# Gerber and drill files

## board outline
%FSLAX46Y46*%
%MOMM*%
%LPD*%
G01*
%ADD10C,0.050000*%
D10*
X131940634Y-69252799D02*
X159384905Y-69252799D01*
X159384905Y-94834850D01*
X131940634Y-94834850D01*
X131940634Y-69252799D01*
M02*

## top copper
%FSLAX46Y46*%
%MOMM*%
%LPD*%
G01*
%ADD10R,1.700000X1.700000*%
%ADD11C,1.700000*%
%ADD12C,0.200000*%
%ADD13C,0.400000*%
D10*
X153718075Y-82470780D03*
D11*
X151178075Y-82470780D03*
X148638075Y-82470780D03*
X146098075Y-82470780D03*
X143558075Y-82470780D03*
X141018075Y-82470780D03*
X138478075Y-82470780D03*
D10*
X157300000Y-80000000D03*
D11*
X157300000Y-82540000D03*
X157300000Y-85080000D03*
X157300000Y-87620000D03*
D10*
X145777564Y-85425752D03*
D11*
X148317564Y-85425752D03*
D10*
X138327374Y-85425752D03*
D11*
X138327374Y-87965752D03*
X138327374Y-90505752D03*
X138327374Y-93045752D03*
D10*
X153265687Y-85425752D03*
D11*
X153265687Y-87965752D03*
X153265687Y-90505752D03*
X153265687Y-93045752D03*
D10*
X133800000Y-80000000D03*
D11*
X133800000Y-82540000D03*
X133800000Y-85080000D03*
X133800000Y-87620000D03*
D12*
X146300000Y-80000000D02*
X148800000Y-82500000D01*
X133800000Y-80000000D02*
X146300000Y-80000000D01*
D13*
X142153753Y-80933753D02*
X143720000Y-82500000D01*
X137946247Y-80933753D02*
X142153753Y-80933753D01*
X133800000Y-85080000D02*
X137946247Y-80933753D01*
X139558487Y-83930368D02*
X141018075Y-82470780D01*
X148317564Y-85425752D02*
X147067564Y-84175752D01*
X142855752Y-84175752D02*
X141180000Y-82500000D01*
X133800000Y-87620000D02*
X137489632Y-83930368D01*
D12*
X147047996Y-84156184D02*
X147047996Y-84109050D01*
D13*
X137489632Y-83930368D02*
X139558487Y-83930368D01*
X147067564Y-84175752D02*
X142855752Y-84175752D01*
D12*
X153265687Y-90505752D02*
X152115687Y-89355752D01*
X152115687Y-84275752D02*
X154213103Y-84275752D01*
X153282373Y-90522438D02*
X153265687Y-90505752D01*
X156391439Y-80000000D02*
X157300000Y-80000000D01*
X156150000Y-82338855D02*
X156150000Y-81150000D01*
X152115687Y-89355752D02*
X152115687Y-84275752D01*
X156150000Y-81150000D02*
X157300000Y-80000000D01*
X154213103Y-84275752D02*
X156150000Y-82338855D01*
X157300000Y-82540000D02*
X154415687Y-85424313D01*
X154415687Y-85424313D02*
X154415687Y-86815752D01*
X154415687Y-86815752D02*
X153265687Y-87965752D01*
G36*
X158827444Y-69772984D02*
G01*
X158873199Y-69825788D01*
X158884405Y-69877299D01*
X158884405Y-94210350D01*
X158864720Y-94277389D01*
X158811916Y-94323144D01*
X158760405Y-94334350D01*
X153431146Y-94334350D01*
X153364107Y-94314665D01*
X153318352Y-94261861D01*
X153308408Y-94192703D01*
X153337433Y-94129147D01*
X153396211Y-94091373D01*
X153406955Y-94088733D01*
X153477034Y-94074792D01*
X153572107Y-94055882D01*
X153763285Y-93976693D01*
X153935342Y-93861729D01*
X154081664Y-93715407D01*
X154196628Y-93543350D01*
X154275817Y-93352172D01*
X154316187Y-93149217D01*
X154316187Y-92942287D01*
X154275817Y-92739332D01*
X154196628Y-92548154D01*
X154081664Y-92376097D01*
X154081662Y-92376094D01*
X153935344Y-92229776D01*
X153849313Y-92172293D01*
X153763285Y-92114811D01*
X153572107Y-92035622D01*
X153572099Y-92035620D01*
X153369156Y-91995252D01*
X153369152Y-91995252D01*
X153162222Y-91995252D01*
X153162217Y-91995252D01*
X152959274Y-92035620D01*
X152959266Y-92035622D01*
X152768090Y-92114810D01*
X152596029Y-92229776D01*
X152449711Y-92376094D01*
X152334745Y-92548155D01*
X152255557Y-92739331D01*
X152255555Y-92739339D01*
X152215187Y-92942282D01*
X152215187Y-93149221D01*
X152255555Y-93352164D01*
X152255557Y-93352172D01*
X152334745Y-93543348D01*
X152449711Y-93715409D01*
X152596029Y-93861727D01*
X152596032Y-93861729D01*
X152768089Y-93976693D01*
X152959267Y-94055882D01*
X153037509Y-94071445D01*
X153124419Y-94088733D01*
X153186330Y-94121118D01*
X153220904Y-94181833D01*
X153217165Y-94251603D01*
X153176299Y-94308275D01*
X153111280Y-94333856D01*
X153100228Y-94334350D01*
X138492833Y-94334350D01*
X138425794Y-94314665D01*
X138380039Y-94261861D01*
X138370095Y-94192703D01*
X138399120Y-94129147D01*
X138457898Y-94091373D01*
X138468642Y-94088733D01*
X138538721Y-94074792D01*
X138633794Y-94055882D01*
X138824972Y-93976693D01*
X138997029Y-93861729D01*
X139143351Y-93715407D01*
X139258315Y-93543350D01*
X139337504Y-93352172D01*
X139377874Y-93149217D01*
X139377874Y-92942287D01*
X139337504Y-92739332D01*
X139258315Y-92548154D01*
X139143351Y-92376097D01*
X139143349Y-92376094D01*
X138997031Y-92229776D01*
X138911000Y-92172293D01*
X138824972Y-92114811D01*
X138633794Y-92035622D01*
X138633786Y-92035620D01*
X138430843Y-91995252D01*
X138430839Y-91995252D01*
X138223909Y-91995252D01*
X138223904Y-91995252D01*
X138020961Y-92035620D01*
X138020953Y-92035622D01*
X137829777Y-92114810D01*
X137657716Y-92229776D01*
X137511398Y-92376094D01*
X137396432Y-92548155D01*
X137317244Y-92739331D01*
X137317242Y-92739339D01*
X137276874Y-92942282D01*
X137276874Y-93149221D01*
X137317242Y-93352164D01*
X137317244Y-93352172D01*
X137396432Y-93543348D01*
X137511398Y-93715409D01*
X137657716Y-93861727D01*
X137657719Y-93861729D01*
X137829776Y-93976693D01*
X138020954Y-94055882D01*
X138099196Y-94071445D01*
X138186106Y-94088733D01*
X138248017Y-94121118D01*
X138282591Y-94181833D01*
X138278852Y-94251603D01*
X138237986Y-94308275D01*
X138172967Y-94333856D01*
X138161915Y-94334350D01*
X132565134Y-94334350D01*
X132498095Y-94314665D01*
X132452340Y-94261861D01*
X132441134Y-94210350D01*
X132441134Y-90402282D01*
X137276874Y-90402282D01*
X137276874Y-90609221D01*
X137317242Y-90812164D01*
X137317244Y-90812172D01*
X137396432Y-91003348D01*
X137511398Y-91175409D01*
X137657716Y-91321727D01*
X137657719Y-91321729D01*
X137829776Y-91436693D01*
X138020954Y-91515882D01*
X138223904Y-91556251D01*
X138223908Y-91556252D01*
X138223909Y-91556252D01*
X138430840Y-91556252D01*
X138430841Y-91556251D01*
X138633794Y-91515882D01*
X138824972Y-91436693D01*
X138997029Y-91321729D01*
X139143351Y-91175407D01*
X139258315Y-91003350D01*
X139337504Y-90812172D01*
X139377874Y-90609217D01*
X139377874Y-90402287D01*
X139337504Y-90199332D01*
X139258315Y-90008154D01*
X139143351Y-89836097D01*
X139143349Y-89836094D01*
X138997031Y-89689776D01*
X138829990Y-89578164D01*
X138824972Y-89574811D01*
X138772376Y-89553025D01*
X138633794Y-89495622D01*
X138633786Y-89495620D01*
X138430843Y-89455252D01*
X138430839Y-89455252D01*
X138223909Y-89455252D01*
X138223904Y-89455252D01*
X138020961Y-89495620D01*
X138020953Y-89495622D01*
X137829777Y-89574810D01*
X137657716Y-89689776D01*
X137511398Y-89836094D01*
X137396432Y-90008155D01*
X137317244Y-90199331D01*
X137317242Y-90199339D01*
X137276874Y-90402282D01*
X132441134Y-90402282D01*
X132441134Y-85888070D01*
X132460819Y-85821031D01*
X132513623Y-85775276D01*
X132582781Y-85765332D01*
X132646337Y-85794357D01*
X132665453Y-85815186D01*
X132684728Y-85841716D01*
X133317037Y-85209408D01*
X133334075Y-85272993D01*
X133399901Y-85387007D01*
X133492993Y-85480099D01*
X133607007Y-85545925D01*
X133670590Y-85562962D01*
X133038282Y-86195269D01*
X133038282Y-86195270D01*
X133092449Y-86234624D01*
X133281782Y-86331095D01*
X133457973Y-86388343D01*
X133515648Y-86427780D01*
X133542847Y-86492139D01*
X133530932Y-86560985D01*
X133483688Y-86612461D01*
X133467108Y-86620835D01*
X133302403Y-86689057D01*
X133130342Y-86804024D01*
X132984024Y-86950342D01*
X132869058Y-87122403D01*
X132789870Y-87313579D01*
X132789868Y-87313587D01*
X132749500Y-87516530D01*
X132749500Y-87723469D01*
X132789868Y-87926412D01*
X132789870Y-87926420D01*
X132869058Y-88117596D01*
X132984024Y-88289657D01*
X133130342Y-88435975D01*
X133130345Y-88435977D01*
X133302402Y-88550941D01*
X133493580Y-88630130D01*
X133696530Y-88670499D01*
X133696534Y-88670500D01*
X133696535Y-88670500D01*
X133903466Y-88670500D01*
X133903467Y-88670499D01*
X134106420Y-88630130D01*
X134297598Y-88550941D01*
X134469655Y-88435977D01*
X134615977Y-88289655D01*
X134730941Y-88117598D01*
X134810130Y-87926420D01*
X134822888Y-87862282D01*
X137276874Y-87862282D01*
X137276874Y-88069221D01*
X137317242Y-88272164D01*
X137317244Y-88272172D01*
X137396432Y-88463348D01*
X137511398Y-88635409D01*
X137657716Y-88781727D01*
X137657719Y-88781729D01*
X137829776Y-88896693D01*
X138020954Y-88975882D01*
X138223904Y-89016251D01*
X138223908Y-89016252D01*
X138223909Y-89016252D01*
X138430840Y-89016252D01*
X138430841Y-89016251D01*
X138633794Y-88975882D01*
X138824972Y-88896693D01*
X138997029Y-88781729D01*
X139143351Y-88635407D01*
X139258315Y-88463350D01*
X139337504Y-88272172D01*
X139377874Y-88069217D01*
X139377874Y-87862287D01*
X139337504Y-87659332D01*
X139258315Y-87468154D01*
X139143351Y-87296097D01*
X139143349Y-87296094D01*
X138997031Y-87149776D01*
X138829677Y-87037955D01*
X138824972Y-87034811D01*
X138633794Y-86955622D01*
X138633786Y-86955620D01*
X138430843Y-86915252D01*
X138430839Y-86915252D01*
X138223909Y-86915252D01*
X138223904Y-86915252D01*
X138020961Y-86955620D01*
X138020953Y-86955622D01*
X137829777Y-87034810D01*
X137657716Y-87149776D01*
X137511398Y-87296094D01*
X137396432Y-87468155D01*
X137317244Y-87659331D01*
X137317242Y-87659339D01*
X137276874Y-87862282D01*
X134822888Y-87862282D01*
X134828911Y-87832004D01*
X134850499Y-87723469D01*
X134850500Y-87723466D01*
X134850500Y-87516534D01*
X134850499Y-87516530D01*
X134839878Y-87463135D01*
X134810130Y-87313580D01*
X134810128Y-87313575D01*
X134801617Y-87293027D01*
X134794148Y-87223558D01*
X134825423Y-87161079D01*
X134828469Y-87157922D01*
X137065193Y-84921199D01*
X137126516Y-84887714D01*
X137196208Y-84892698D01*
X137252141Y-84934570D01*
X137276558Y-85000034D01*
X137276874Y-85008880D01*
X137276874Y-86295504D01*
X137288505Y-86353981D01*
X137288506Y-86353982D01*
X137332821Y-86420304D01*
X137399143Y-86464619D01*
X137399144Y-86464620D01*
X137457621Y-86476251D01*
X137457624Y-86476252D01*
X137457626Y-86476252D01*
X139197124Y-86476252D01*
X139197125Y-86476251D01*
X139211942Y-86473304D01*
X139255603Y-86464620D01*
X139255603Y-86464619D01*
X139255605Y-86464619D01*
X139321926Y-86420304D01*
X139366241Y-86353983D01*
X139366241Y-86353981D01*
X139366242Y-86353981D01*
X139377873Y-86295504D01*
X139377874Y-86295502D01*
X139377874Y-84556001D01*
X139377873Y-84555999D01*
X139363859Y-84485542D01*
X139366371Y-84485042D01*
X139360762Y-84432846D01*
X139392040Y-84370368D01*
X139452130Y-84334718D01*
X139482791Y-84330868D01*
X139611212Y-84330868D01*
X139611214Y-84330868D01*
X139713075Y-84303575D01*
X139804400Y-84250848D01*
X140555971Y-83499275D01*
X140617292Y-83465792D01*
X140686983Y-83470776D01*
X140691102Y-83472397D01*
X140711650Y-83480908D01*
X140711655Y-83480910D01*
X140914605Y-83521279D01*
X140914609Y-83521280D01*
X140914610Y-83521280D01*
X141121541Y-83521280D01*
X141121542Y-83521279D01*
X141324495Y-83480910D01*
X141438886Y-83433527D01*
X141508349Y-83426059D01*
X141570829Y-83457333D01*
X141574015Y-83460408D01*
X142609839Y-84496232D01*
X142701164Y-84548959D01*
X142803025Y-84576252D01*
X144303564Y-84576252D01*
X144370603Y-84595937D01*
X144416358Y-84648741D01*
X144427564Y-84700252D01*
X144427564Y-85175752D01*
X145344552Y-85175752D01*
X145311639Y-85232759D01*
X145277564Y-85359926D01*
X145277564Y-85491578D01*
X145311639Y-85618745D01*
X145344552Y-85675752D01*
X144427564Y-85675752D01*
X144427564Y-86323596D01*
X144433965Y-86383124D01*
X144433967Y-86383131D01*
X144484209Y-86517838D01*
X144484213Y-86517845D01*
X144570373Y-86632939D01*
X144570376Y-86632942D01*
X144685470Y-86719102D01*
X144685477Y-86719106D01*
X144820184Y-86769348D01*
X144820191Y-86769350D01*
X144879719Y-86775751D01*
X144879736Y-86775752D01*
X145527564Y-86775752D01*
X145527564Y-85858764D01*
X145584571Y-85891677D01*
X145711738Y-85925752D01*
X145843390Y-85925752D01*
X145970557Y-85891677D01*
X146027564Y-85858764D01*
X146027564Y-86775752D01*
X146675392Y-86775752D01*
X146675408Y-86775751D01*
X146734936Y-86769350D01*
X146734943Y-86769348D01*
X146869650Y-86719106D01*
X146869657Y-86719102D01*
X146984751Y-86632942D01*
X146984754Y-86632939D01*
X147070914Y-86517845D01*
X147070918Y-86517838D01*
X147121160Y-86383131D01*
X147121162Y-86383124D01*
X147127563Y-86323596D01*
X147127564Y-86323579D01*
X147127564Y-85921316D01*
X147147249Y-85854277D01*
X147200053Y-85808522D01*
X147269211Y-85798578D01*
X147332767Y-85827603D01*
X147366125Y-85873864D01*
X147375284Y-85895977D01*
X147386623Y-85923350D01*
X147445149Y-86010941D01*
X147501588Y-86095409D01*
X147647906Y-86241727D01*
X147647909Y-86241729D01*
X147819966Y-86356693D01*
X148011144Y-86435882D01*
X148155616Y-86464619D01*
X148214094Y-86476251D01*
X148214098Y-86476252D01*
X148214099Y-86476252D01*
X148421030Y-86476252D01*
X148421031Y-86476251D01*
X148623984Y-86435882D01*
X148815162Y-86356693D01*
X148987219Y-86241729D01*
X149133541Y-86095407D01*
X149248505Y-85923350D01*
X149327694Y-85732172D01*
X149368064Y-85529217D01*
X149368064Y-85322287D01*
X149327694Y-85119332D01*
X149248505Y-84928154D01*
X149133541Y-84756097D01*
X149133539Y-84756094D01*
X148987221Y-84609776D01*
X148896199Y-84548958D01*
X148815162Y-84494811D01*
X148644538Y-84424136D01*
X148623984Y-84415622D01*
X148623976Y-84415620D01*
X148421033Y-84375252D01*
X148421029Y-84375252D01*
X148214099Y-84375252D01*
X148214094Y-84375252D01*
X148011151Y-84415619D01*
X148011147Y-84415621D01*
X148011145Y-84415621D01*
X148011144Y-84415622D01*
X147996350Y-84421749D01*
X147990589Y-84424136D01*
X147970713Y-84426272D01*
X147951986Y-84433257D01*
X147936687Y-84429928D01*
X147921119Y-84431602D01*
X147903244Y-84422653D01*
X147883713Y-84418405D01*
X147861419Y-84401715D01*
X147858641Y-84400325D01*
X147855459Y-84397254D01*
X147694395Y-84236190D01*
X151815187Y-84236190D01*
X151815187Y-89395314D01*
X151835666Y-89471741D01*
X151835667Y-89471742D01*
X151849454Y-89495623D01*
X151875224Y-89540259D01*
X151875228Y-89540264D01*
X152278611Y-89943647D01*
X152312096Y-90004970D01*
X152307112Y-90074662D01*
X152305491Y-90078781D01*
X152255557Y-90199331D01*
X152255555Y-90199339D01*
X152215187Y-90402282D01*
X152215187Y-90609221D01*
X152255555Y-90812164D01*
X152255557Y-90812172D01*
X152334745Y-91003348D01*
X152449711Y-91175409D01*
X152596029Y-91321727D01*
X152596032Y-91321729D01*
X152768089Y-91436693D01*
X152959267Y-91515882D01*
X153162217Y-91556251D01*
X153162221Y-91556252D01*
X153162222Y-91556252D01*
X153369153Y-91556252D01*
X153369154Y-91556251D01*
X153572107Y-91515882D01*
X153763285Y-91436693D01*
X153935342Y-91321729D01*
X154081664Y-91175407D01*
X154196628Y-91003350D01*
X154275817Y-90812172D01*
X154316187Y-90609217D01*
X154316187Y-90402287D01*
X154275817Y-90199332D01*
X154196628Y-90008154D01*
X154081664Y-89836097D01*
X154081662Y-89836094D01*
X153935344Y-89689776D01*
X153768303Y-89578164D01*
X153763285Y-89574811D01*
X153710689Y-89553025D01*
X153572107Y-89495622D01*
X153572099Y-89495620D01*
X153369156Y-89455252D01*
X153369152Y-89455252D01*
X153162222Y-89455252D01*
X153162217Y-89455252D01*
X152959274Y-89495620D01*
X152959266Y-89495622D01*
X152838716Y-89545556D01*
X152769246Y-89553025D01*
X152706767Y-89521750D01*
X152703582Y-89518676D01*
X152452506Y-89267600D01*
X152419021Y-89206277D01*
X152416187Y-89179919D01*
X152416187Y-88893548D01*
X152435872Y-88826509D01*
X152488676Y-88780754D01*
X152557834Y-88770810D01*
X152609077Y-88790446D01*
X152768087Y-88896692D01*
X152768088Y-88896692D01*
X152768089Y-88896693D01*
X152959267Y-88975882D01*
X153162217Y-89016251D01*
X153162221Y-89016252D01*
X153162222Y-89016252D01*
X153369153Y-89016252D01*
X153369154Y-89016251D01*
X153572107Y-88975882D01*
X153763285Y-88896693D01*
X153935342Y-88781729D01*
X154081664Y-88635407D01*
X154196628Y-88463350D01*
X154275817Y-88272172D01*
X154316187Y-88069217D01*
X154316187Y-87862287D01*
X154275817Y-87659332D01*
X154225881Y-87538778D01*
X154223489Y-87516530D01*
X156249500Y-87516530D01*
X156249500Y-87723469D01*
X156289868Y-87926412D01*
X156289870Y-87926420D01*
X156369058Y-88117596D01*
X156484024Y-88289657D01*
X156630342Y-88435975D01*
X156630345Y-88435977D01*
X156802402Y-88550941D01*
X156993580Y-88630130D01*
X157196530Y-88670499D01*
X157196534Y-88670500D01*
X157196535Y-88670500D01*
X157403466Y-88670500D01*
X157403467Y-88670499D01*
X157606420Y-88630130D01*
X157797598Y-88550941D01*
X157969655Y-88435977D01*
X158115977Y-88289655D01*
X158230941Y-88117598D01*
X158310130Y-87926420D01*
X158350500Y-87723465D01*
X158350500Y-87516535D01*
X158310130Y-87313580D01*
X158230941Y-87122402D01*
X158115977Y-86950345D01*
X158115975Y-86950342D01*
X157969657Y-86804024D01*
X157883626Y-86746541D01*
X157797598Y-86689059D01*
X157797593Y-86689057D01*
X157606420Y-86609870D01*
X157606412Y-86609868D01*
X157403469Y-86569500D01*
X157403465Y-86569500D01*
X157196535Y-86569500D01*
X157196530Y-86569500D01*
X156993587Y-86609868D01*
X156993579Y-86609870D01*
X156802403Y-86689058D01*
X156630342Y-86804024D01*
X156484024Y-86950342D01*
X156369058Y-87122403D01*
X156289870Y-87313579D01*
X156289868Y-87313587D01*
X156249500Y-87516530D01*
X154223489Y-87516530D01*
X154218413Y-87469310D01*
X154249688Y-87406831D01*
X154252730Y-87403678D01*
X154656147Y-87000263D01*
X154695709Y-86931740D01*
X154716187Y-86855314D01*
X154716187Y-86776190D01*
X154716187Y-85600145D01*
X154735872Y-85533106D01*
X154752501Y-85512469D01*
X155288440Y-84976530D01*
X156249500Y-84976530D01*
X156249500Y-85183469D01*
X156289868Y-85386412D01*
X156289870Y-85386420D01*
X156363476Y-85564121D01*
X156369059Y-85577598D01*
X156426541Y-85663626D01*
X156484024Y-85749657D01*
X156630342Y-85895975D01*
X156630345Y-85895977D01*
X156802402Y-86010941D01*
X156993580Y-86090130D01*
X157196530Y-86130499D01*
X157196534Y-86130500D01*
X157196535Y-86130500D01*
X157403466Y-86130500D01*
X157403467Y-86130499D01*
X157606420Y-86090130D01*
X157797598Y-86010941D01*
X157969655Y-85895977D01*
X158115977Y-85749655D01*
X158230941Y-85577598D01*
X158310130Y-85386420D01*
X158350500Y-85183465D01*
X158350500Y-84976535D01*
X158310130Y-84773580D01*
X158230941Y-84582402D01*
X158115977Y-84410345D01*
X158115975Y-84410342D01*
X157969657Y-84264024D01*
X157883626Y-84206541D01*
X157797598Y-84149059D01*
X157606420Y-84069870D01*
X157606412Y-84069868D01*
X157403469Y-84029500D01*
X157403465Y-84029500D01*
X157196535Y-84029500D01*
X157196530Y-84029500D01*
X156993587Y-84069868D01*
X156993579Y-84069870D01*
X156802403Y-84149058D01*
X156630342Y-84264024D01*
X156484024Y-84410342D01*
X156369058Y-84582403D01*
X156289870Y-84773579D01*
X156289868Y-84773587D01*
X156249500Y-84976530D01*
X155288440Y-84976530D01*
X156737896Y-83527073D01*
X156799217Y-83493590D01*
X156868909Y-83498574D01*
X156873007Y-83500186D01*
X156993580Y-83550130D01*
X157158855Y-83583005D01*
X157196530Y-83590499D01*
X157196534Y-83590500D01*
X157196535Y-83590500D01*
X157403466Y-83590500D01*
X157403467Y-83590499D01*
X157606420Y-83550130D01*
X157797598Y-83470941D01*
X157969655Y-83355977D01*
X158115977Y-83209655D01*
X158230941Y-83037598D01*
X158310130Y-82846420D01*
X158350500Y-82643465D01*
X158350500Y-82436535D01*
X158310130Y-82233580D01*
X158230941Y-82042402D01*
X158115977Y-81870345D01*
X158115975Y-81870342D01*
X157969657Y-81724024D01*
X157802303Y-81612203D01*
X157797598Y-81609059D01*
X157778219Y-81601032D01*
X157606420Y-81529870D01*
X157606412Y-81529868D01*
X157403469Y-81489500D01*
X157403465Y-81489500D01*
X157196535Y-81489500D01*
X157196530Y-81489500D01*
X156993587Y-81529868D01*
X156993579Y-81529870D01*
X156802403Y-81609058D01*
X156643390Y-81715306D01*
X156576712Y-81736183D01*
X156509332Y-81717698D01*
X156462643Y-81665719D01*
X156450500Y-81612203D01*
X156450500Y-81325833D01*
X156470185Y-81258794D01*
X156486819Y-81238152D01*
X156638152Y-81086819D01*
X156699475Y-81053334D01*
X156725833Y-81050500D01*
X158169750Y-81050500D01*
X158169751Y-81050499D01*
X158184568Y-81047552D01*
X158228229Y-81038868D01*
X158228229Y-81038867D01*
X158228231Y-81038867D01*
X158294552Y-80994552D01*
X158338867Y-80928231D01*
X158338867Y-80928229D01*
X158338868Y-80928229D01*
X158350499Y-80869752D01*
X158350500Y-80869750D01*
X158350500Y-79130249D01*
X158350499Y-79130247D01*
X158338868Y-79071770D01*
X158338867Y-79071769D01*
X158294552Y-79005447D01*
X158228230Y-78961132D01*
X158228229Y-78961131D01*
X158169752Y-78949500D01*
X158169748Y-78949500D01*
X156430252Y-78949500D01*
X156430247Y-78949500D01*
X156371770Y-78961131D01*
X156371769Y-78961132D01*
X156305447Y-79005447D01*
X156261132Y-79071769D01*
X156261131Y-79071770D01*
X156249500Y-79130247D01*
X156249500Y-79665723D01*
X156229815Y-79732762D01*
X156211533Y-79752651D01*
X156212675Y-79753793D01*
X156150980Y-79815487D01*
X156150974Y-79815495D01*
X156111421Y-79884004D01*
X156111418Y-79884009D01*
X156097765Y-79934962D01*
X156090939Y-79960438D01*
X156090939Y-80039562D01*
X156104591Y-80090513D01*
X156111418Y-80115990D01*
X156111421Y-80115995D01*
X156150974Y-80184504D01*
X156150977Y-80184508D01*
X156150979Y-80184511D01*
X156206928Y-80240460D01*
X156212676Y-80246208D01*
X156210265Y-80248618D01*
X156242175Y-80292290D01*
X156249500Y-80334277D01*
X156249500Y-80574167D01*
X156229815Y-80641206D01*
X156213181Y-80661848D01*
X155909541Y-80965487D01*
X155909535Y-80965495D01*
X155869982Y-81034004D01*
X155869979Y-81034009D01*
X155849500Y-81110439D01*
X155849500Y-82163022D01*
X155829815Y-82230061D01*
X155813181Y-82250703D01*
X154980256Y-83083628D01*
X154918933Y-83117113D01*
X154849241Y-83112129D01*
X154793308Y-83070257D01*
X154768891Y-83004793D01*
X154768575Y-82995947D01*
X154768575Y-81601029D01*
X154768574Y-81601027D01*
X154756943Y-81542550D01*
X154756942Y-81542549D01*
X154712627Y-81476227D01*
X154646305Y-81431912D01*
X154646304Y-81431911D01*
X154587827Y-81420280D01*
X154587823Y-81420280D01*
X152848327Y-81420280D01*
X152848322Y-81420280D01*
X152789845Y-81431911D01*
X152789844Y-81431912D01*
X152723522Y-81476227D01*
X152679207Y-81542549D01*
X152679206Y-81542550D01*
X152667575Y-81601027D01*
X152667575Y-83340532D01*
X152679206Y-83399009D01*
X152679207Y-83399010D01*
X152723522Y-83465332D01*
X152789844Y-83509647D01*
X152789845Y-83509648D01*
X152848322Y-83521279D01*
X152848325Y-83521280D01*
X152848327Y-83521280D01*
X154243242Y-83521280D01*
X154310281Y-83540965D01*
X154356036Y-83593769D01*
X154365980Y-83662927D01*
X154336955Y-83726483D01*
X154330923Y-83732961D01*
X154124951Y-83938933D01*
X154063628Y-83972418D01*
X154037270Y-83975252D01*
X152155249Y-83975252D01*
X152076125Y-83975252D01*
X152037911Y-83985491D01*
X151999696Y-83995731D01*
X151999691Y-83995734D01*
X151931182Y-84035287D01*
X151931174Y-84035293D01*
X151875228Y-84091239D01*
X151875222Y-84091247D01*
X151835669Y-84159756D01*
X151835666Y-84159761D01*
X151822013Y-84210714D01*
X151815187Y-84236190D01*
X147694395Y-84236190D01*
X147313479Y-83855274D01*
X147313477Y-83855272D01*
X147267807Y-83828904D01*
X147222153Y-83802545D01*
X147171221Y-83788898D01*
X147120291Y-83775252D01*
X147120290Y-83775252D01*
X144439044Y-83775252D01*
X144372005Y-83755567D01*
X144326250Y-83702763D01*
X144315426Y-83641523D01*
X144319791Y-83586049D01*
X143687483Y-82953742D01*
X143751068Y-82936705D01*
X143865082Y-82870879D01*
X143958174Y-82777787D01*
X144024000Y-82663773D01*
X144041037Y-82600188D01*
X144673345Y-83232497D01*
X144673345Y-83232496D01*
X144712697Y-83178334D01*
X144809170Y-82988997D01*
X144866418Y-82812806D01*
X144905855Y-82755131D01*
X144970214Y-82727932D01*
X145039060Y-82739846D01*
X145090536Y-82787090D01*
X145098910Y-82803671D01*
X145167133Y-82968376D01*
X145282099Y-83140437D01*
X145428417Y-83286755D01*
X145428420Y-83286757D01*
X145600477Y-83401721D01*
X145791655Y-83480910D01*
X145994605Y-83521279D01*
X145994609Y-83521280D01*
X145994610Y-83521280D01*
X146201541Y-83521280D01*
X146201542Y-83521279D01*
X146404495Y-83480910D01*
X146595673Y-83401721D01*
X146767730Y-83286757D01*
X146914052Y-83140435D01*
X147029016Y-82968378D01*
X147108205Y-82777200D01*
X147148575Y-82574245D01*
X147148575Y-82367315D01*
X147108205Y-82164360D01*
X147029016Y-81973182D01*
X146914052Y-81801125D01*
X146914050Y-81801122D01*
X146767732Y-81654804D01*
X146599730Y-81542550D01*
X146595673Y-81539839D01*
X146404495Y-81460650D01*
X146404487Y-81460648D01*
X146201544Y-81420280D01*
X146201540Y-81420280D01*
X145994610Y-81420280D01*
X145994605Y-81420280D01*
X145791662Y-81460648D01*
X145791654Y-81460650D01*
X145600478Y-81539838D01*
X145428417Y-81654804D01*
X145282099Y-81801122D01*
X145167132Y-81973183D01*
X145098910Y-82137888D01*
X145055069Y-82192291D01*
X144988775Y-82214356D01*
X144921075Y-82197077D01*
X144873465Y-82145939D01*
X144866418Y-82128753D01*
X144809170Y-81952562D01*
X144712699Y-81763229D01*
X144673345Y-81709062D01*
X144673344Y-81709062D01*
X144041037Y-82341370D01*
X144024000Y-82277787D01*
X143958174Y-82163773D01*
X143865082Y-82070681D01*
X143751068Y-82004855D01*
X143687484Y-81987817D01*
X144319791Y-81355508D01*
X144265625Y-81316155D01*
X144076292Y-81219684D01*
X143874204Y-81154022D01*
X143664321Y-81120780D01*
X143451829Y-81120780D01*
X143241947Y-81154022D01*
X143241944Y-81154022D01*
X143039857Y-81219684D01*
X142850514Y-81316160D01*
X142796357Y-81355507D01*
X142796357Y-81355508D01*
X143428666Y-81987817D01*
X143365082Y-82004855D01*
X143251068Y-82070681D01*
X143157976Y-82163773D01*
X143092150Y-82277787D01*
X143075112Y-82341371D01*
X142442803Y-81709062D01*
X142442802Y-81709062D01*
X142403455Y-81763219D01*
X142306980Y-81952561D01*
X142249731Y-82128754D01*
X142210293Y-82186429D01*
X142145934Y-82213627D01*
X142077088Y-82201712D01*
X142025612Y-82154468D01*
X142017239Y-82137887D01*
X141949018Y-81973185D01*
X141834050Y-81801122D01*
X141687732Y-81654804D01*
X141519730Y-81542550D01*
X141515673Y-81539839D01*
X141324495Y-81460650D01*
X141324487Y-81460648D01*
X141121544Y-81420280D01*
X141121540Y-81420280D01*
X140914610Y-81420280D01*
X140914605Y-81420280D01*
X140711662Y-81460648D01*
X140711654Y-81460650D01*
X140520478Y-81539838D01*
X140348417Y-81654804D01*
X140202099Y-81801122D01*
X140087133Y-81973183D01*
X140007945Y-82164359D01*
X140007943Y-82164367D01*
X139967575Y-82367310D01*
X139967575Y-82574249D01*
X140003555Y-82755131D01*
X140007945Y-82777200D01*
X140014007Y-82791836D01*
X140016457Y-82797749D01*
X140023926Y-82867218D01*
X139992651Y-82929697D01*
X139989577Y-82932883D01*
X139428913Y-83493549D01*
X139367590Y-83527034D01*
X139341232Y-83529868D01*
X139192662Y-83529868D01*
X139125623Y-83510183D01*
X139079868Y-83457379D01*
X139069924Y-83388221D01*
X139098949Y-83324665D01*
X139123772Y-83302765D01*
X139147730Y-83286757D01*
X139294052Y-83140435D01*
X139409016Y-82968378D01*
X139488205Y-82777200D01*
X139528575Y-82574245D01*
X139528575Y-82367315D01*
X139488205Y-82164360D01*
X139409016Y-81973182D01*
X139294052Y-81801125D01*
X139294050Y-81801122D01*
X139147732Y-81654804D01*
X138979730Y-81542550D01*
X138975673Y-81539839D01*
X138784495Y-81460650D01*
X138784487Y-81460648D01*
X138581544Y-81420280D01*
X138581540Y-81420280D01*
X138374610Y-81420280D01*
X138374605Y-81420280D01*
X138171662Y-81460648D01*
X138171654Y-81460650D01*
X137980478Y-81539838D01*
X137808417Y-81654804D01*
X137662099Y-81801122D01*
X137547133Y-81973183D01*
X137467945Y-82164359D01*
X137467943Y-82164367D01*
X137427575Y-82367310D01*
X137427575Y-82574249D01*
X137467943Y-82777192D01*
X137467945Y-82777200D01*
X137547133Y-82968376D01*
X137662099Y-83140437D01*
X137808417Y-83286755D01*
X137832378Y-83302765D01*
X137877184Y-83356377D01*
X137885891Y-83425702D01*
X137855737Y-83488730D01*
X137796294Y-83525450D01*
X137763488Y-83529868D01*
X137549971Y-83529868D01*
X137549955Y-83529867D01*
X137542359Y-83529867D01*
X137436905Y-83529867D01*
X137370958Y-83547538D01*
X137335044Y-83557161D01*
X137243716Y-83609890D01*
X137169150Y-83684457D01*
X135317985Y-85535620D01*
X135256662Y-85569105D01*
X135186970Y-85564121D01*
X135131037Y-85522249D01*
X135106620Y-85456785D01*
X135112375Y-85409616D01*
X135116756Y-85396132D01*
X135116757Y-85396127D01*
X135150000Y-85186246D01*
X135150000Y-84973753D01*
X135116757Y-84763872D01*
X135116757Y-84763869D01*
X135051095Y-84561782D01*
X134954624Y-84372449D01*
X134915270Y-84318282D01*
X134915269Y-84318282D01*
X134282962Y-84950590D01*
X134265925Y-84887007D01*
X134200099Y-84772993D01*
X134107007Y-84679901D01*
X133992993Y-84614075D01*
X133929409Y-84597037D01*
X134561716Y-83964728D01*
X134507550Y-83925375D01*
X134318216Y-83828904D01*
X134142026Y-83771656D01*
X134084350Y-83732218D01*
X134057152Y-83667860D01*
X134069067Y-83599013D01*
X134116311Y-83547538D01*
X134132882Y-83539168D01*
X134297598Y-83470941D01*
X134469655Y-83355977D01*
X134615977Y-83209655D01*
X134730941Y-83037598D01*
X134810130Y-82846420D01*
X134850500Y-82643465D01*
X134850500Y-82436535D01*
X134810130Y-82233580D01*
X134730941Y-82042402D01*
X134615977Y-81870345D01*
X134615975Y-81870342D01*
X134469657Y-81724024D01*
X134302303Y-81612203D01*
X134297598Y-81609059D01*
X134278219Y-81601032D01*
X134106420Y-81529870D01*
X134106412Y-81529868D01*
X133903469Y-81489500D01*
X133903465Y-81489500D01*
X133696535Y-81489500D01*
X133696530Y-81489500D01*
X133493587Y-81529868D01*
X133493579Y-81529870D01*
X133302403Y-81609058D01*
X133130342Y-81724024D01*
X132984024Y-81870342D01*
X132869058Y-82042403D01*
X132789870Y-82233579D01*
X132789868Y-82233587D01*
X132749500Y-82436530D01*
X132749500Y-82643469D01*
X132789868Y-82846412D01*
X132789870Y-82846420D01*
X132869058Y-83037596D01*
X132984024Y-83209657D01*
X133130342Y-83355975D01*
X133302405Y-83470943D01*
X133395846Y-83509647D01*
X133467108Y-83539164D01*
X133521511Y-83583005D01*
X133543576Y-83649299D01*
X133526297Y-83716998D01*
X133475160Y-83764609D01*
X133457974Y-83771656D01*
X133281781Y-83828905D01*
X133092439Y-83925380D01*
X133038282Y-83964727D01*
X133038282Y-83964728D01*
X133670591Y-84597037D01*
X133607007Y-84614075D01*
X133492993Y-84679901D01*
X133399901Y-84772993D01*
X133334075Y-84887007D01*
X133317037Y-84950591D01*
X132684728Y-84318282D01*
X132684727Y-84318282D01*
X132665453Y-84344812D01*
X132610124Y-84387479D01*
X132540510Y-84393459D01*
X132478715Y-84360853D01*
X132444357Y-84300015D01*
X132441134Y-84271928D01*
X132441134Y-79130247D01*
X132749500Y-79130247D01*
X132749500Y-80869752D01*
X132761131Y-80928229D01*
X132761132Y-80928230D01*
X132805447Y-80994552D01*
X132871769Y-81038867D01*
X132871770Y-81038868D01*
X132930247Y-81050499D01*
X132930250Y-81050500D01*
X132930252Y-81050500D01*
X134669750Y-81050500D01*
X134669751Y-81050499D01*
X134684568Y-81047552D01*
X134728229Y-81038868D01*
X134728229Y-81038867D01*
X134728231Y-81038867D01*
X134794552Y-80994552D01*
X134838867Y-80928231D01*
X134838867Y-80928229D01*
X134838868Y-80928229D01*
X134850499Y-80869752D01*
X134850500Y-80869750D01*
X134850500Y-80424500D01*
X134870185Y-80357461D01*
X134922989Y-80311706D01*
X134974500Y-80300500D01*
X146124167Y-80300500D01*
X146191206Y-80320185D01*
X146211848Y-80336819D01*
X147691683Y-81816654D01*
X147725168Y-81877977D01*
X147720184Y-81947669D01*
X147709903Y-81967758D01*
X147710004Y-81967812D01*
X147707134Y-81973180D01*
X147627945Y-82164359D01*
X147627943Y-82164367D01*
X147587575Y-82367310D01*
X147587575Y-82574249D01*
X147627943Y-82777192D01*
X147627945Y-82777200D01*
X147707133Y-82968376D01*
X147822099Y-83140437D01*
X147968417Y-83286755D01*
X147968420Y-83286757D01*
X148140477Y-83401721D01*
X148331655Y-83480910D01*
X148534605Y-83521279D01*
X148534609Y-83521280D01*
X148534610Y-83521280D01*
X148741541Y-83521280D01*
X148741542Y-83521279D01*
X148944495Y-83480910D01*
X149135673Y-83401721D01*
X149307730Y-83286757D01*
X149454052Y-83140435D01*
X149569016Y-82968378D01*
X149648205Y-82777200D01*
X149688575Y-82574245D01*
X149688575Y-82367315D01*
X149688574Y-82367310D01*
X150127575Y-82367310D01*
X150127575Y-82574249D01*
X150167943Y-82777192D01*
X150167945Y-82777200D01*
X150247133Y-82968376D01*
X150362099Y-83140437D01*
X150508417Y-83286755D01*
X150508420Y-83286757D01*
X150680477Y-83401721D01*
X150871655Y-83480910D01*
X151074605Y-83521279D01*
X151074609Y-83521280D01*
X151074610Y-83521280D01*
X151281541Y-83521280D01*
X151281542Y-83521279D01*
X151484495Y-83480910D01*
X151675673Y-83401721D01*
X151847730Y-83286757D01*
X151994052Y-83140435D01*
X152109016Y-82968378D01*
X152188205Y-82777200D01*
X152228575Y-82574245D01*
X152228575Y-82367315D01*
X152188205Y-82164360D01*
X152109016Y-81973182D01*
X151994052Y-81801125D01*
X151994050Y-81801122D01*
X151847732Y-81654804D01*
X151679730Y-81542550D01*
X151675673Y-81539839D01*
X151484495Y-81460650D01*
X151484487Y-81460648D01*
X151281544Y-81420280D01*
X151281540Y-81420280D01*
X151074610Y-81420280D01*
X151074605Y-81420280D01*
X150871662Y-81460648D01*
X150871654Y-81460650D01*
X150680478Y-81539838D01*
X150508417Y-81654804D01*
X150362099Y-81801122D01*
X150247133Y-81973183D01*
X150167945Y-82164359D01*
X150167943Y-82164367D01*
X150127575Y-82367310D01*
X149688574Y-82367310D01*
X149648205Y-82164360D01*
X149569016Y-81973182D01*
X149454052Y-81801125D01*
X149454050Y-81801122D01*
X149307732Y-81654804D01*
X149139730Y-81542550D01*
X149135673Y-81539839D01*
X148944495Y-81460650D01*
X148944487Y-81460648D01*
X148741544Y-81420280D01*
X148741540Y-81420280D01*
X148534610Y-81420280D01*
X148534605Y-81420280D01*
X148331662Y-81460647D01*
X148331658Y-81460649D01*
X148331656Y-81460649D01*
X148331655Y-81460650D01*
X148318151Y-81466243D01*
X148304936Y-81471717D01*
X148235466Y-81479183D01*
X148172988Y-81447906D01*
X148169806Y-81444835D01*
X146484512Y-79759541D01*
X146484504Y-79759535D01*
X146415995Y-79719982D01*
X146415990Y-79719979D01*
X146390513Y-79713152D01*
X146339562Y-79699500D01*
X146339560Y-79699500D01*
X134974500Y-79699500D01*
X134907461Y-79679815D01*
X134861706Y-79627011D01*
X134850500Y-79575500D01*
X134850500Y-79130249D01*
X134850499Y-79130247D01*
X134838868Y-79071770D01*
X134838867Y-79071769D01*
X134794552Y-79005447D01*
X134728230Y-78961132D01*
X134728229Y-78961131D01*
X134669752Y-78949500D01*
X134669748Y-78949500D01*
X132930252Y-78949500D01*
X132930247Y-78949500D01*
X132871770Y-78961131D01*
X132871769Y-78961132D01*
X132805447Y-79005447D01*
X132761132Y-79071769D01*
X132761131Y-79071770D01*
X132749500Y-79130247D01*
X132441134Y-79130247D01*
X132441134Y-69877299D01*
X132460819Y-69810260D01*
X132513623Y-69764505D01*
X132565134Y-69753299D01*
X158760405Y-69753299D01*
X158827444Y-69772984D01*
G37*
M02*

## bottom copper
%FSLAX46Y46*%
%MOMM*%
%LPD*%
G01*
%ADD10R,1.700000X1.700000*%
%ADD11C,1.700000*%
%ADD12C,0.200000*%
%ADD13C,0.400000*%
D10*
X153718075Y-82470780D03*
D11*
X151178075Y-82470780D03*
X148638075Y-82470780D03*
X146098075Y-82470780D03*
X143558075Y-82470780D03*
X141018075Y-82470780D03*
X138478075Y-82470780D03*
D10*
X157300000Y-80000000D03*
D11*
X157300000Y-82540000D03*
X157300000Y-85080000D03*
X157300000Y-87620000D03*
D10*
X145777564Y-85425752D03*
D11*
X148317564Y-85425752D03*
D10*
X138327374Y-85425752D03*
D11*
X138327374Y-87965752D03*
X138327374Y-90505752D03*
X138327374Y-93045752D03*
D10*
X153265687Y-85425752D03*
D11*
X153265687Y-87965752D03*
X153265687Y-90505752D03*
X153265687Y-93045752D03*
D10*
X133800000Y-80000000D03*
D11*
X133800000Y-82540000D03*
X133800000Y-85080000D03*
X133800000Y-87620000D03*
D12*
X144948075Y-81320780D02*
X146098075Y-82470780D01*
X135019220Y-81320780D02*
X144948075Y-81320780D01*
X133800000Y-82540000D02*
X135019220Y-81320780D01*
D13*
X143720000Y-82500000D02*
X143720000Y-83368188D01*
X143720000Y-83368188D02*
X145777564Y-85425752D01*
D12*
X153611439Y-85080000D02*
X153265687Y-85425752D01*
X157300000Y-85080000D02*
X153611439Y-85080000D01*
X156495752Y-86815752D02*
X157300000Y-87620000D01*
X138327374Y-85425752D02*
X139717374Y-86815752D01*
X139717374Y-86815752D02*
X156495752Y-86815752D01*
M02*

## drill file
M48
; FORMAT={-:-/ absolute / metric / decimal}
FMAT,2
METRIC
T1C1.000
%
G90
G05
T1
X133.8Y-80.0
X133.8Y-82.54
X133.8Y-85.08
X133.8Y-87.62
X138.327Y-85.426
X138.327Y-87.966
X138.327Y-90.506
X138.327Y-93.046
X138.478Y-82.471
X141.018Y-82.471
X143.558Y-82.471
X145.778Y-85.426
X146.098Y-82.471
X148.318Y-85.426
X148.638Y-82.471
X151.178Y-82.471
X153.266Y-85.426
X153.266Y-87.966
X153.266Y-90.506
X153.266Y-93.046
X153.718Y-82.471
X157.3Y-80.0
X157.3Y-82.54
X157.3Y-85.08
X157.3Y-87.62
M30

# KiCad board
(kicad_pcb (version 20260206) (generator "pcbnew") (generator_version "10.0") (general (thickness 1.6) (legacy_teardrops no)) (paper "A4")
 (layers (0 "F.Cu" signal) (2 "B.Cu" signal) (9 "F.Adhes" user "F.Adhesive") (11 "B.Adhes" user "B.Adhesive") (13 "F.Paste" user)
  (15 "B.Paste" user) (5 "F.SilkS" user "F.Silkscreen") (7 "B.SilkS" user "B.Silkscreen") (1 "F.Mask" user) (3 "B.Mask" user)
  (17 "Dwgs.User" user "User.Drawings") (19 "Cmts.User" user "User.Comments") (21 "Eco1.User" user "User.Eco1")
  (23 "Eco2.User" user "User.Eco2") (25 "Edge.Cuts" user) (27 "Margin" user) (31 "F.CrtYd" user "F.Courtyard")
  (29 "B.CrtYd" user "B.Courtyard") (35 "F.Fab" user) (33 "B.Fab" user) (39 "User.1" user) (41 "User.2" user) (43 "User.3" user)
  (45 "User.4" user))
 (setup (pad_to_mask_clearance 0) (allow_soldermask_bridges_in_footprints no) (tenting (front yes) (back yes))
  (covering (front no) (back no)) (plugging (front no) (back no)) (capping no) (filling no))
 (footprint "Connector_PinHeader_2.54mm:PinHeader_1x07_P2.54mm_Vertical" (layer "F.Cu") (at 153.718075 82.47078 -90)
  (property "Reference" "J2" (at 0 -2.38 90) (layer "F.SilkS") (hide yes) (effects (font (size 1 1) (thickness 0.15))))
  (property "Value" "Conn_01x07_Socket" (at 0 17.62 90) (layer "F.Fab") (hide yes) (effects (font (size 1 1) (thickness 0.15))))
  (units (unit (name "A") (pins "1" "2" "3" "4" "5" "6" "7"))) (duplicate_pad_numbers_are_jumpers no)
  (pad "1" thru_hole rect (at 0 0 270) (size 1.7 1.7) (drill 1) (layers "*.Cu" "*.Mask") (remove_unused_layers no)
   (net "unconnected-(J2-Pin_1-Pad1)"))
  (pad "2" thru_hole circle (at 0 2.54 270) (size 1.7 1.7) (drill 1) (layers "*.Cu" "*.Mask") (remove_unused_layers no)
   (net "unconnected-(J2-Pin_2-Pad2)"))
  (pad "3" thru_hole circle (at 0 5.08 270) (size 1.7 1.7) (drill 1) (layers "*.Cu" "*.Mask") (remove_unused_layers no) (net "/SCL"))
  (pad "4" thru_hole circle (at 0 7.62 270) (size 1.7 1.7) (drill 1) (layers "*.Cu" "*.Mask") (remove_unused_layers no) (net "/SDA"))
  (pad "5" thru_hole circle (at 0 10.16 270) (size 1.7 1.7) (drill 1) (layers "*.Cu" "*.Mask") (remove_unused_layers no) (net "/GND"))
  (pad "6" thru_hole circle (at 0 12.7 270) (size 1.7 1.7) (drill 1) (layers "*.Cu" "*.Mask") (remove_unused_layers no) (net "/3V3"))
  (pad "7" thru_hole circle (at 0 15.24 270) (size 1.7 1.7) (drill 1) (layers "*.Cu" "*.Mask") (remove_unused_layers no)
   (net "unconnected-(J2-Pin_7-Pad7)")))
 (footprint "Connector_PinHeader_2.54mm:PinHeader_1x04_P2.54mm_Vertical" (layer "F.Cu") (at 157.3 80)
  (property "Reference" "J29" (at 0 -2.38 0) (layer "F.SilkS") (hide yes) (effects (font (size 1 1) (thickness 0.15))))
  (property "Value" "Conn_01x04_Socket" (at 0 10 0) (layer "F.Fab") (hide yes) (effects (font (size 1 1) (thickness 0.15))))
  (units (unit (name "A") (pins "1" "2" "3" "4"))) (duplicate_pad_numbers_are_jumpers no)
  (pad "1" thru_hole rect (at 0 0) (size 1.7 1.7) (drill 1) (layers "*.Cu" "*.Mask") (remove_unused_layers no) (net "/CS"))
  (pad "2" thru_hole circle (at 0 2.54) (size 1.7 1.7) (drill 1) (layers "*.Cu" "*.Mask") (remove_unused_layers no) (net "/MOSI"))
  (pad "3" thru_hole circle (at 0 5.08) (size 1.7 1.7) (drill 1) (layers "*.Cu" "*.Mask") (remove_unused_layers no) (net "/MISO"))
  (pad "4" thru_hole circle (at 0 7.62) (size 1.7 1.7) (drill 1) (layers "*.Cu" "*.Mask") (remove_unused_layers no) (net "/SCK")))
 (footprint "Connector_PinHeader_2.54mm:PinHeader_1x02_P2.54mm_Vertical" (layer "F.Cu") (at 145.777564 85.425752 90)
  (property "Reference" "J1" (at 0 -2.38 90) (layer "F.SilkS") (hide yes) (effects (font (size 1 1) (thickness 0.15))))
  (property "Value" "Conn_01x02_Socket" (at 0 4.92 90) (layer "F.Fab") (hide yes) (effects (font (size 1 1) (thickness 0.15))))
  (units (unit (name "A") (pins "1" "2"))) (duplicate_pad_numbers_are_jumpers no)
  (pad "1" thru_hole rect (at 0 0 90) (size 1.7 1.7) (drill 1) (layers "*.Cu" "*.Mask") (remove_unused_layers no) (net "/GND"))
  (pad "2" thru_hole circle (at 0 2.54 90) (size 1.7 1.7) (drill 1) (layers "*.Cu" "*.Mask") (remove_unused_layers no) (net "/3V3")))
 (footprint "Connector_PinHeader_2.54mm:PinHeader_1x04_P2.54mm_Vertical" (layer "F.Cu") (at 138.327374 85.425752)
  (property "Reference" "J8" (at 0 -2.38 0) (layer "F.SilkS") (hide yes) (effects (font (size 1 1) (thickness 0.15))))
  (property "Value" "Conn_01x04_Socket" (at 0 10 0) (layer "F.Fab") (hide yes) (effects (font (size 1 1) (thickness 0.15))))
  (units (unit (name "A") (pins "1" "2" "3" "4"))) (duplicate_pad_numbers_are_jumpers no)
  (pad "1" thru_hole rect (at 0 0) (size 1.7 1.7) (drill 1) (layers "*.Cu" "*.Mask") (remove_unused_layers no) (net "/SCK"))
  (pad "2" thru_hole circle (at 0 2.54) (size 1.7 1.7) (drill 1) (layers "*.Cu" "*.Mask") (remove_unused_layers no)
   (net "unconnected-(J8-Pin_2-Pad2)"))
  (pad "3" thru_hole circle (at 0 5.08) (size 1.7 1.7) (drill 1) (layers "*.Cu" "*.Mask") (remove_unused_layers no)
   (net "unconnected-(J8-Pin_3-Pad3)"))
  (pad "4" thru_hole circle (at 0 7.62) (size 1.7 1.7) (drill 1) (layers "*.Cu" "*.Mask") (remove_unused_layers no)
   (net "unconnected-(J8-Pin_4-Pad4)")))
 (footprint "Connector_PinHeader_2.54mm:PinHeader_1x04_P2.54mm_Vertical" (layer "F.Cu") (at 153.265687 85.425752)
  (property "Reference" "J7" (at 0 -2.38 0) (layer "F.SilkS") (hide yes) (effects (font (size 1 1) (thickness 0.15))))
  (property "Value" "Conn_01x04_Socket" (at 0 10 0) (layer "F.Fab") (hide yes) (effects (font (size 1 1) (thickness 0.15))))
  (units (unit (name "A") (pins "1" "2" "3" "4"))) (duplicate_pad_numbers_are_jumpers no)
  (pad "1" thru_hole rect (at 0 0) (size 1.7 1.7) (drill 1) (layers "*.Cu" "*.Mask") (remove_unused_layers no) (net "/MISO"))
  (pad "2" thru_hole circle (at 0 2.54) (size 1.7 1.7) (drill 1) (layers "*.Cu" "*.Mask") (remove_unused_layers no) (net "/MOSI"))
  (pad "3" thru_hole circle (at 0 5.08) (size 1.7 1.7) (drill 1) (layers "*.Cu" "*.Mask") (remove_unused_layers no) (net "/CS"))
  (pad "4" thru_hole circle (at 0 7.62) (size 1.7 1.7) (drill 1) (layers "*.Cu" "*.Mask") (remove_unused_layers no)
   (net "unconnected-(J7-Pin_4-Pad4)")))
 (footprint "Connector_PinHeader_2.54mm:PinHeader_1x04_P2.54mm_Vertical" (layer "F.Cu") (at 133.8 80)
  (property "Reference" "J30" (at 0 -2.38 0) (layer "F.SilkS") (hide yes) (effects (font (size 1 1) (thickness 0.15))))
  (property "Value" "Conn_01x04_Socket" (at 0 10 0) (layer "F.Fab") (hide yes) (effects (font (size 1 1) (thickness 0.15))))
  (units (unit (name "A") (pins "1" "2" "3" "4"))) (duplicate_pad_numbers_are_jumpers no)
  (pad "1" thru_hole rect (at 0 0) (size 1.7 1.7) (drill 1) (layers "*.Cu" "*.Mask") (remove_unused_layers no) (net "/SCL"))
  (pad "2" thru_hole circle (at 0 2.54) (size 1.7 1.7) (drill 1) (layers "*.Cu" "*.Mask") (remove_unused_layers no) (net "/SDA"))
  (pad "3" thru_hole circle (at 0 5.08) (size 1.7 1.7) (drill 1) (layers "*.Cu" "*.Mask") (remove_unused_layers no) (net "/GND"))
  (pad "4" thru_hole circle (at 0 7.62) (size 1.7 1.7) (drill 1) (layers "*.Cu" "*.Mask") (remove_unused_layers no) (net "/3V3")))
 (gr_rect (start 131.940634 69.252799) (end 159.384905 94.83485) (stroke (width 0.05) (type default)) (fill no) (layer "Edge.Cuts"))
 (segment (start 146.3 80) (end 148.8 82.5) (width 0.2) (layer "F.Cu") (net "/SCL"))
 (segment (start 133.8 80) (end 146.3 80) (width 0.2) (layer "F.Cu") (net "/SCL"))
 (segment (start 144.948075 81.32078) (end 146.098075 82.47078) (width 0.2) (layer "B.Cu") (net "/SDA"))
 (segment (start 135.01922 81.32078) (end 144.948075 81.32078) (width 0.2) (layer "B.Cu") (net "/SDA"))
 (segment (start 133.8 82.54) (end 135.01922 81.32078) (width 0.2) (layer "B.Cu") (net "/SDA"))
 (segment (start 142.153753 80.933753) (end 143.72 82.5) (width 0.4) (layer "F.Cu") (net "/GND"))
 (segment (start 137.946247 80.933753) (end 142.153753 80.933753) (width 0.4) (layer "F.Cu") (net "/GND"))
 (segment (start 133.8 85.08) (end 137.946247 80.933753) (width 0.4) (layer "F.Cu") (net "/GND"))
 (segment (start 143.72 82.5) (end 143.72 83.368188) (width 0.4) (layer "B.Cu") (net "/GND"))
 (segment (start 143.72 83.368188) (end 145.777564 85.425752) (width 0.4) (layer "B.Cu") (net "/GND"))
 (segment (start 139.558487 83.930368) (end 141.018075 82.47078) (width 0.4) (layer "F.Cu") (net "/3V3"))
 (segment (start 148.317564 85.425752) (end 147.067564 84.175752) (width 0.4) (layer "F.Cu") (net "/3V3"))
 (segment (start 142.855752 84.175752) (end 141.18 82.5) (width 0.4) (layer "F.Cu") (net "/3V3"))
 (segment (start 133.8 87.62) (end 137.489632 83.930368) (width 0.4) (layer "F.Cu") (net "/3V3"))
 (segment (start 147.047996 84.156184) (end 147.047996 84.10905) (width 0.2) (layer "F.Cu") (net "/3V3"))
 (segment (start 137.489632 83.930368) (end 139.558487 83.930368) (width 0.4) (layer "F.Cu") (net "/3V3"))
 (segment (start 147.067564 84.175752) (end 142.855752 84.175752) (width 0.4) (layer "F.Cu") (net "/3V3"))
 (segment (start 153.265687 90.505752) (end 152.115687 89.355752) (width 0.2) (layer "F.Cu") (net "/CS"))
 (segment (start 152.115687 84.275752) (end 154.213103 84.275752) (width 0.2) (layer "F.Cu") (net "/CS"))
 (segment (start 153.282373 90.522438) (end 153.265687 90.505752) (width 0.2) (layer "F.Cu") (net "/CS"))
 (segment (start 156.391439 80) (end 157.3 80) (width 0.2) (layer "F.Cu") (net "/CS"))
 (segment (start 156.15 82.338855) (end 156.15 81.15) (width 0.2) (layer "F.Cu") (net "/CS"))
 (segment (start 152.115687 89.355752) (end 152.115687 84.275752) (width 0.2) (layer "F.Cu") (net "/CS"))
 (segment (start 156.15 81.15) (end 157.3 80) (width 0.2) (layer "F.Cu") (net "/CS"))
 (segment (start 154.213103 84.275752) (end 156.15 82.338855) (width 0.2) (layer "F.Cu") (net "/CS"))
 (segment (start 157.3 82.54) (end 154.415687 85.424313) (width 0.2) (layer "F.Cu") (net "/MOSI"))
 (segment (start 154.415687 85.424313) (end 154.415687 86.815752) (width 0.2) (layer "F.Cu") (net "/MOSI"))
 (segment (start 154.415687 86.815752) (end 153.265687 87.965752) (width 0.2) (layer "F.Cu") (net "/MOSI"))
 (segment (start 153.611439 85.08) (end 153.265687 85.425752) (width 0.2) (layer "B.Cu") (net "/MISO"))
 (segment (start 157.3 85.08) (end 153.611439 85.08) (width 0.2) (layer "B.Cu") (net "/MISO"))
 (segment (start 156.495752 86.815752) (end 157.3 87.62) (width 0.2) (layer "B.Cu") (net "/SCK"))
 (segment (start 138.327374 85.425752) (end 139.717374 86.815752) (width 0.2) (layer "B.Cu") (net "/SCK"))
 (segment (start 139.717374 86.815752) (end 156.495752 86.815752) (width 0.2) (layer "B.Cu") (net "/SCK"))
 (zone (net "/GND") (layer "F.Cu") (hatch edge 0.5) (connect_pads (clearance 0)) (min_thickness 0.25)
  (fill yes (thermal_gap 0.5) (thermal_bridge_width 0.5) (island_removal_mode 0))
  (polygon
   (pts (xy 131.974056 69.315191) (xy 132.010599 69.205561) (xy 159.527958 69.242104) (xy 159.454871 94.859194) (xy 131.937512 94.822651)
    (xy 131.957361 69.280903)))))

